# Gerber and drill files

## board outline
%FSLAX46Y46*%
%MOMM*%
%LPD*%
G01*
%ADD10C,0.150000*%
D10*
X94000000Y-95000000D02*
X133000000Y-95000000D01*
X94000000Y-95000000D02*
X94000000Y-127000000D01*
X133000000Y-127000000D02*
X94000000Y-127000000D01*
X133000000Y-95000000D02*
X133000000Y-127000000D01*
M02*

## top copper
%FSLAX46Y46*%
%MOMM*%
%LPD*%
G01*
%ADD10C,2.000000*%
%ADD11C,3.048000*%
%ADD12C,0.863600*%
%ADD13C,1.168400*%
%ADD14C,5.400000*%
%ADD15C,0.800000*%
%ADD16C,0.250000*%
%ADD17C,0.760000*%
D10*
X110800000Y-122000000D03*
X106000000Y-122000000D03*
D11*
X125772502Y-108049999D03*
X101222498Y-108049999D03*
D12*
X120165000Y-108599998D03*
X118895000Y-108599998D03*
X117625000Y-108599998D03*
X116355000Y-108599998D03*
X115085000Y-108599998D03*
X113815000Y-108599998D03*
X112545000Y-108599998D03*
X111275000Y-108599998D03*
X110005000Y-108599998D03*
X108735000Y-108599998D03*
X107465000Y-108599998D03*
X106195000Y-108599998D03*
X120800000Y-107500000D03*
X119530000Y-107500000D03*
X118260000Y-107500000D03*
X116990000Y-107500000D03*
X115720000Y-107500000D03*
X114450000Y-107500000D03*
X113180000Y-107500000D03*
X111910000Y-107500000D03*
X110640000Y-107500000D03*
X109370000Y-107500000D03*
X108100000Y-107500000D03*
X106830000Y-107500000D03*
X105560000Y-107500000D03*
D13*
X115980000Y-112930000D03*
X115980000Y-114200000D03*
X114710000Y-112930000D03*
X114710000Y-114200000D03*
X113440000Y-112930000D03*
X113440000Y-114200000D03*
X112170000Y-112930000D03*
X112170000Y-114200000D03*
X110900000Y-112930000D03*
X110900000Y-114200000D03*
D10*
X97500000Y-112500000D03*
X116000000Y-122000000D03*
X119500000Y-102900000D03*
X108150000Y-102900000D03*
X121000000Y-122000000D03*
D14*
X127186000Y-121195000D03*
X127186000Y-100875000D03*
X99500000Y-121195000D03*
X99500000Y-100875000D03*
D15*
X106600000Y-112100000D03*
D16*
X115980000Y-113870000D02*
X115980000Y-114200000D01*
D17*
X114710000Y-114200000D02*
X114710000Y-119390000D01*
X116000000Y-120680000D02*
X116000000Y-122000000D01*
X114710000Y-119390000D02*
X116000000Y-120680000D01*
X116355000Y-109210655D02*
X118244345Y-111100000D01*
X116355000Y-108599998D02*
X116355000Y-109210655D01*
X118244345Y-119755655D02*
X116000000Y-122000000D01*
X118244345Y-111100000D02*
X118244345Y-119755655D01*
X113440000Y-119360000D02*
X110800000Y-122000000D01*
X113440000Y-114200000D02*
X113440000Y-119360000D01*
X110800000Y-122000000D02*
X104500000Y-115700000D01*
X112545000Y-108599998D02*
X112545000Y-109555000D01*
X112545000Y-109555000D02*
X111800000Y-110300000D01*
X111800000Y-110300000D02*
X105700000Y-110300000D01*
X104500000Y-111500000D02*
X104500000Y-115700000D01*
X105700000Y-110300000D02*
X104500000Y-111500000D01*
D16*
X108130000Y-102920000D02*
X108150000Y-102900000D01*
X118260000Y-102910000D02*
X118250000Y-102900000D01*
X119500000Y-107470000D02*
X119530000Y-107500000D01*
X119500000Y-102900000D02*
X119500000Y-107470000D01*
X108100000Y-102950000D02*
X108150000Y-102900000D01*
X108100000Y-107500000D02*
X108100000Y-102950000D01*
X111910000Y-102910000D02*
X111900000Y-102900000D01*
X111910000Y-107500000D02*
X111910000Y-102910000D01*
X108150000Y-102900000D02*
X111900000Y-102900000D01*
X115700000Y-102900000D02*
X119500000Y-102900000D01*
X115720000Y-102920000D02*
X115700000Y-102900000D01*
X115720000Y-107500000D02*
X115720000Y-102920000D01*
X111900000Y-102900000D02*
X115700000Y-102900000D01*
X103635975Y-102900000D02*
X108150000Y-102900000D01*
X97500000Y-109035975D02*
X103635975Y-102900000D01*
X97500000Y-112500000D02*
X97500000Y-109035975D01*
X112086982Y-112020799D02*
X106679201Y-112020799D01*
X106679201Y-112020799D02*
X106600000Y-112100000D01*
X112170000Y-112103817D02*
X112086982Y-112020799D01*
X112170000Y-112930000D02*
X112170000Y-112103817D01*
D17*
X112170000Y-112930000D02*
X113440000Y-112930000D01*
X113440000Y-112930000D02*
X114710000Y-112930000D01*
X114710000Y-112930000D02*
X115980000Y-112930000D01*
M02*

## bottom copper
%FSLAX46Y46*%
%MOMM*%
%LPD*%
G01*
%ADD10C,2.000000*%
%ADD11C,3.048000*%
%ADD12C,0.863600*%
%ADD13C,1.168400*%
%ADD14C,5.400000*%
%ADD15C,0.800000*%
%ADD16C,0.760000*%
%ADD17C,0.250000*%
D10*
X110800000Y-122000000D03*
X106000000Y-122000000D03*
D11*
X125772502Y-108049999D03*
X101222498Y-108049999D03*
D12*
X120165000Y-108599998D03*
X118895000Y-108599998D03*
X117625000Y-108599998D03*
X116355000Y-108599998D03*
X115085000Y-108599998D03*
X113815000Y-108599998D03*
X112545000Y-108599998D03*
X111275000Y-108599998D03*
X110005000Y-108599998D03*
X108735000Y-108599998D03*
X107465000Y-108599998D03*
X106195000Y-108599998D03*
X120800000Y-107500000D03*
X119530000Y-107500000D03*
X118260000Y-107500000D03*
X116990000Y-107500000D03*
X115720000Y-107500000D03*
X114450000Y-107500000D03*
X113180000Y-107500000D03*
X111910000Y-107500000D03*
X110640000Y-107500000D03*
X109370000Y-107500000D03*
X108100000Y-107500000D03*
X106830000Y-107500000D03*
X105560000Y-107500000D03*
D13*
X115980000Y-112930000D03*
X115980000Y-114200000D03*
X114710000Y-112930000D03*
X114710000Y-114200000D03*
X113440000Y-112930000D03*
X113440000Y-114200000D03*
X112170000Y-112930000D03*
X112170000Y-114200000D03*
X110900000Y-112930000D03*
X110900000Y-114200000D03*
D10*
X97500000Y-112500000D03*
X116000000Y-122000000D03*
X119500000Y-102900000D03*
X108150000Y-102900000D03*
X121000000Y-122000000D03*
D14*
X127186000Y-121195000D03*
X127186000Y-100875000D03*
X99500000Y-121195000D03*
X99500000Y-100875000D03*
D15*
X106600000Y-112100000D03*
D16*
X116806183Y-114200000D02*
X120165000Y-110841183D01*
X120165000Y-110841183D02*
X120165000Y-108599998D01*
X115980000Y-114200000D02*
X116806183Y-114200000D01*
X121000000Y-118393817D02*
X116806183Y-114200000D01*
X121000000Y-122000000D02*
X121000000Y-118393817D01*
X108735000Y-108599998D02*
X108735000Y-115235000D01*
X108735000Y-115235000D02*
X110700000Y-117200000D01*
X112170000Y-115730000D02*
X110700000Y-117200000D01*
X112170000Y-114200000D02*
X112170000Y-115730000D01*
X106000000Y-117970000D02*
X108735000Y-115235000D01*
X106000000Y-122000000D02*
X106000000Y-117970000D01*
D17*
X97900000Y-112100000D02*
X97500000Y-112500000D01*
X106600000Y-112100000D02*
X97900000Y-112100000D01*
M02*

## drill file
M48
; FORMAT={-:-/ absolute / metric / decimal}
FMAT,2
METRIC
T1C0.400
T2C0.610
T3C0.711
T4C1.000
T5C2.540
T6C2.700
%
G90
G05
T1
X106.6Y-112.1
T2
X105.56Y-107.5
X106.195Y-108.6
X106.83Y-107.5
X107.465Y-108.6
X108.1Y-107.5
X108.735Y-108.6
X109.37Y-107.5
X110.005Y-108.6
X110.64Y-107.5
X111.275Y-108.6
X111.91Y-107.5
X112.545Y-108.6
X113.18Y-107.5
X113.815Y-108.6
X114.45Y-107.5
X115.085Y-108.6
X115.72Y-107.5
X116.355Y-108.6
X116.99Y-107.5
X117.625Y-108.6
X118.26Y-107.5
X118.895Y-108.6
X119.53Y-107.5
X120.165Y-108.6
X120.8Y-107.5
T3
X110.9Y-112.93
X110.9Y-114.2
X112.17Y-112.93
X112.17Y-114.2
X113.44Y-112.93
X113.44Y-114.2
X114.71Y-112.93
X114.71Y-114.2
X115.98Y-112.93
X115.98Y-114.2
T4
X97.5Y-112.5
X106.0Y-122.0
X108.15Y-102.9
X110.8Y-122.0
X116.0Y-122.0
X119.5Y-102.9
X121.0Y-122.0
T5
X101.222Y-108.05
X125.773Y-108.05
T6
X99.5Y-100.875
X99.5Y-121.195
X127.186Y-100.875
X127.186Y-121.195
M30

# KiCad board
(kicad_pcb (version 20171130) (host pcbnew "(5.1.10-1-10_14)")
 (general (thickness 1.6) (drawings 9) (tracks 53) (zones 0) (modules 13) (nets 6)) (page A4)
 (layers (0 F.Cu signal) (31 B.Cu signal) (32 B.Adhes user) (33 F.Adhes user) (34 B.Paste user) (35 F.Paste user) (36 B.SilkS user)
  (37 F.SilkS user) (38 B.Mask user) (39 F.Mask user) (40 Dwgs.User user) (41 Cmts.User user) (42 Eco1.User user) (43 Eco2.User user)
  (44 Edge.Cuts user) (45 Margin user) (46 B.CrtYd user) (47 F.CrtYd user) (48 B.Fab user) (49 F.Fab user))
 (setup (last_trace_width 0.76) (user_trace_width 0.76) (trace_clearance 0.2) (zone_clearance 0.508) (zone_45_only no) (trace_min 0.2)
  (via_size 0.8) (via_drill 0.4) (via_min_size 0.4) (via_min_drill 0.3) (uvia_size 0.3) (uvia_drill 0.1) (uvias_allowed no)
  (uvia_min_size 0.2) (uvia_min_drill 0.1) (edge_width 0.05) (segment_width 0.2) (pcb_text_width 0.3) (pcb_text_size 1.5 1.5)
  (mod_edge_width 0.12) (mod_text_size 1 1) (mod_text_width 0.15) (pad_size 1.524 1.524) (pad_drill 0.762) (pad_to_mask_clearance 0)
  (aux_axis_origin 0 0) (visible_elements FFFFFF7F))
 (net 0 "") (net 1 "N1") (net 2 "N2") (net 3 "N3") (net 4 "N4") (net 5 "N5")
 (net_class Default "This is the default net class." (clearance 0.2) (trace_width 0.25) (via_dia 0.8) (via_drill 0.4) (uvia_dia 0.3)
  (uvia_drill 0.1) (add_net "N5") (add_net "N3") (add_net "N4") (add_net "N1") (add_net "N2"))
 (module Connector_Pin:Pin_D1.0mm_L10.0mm (layer F.Cu) (at 110.8 122)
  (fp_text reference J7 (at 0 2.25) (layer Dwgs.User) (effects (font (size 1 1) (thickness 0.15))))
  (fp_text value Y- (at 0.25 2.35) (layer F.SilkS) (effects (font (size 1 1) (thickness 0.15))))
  (pad 1 thru_hole circle (at 0 0) (size 2 2) (drill 1) (layers *.Cu *.Mask) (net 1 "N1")))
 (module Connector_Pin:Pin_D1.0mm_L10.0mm (layer F.Cu) (at 106 122)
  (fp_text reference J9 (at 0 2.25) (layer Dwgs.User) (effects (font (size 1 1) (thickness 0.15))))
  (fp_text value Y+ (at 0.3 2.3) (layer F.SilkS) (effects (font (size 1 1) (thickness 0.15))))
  (pad 1 thru_hole circle (at 0 0) (size 2 2) (drill 1) (layers *.Cu *.Mask) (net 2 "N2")))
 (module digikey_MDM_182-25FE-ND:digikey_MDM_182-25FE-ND (layer F.Cu) (at 120.8 107.5)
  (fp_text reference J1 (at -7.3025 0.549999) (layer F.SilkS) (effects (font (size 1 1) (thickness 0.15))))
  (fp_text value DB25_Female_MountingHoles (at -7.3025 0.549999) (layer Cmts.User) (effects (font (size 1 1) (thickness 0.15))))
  (pad 28 thru_hole circle (at 4.972502 0.549999 90) (size 3.048 3.048) (drill 2.54) (layers *.Cu *.Mask))
  (pad 27 thru_hole circle (at -19.577502 0.549999 90) (size 3.048 3.048) (drill 2.54) (layers *.Cu *.Mask))
  (pad 14 thru_hole circle (at -0.635 1.099998) (size 0.8636 0.8636) (drill 0.6096) (layers *.Cu *.Mask) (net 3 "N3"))
  (pad 15 thru_hole circle (at -1.905 1.099998) (size 0.8636 0.8636) (drill 0.6096) (layers *.Cu *.Mask))
  (pad 16 thru_hole circle (at -3.175 1.099998) (size 0.8636 0.8636) (drill 0.6096) (layers *.Cu *.Mask))
  (pad 17 thru_hole circle (at -4.445 1.099998) (size 0.8636 0.8636) (drill 0.6096) (layers *.Cu *.Mask) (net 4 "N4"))
  (pad 18 thru_hole circle (at -5.715 1.099998) (size 0.8636 0.8636) (drill 0.6096) (layers *.Cu *.Mask))
  (pad 19 thru_hole circle (at -6.985 1.099998) (size 0.8636 0.8636) (drill 0.6096) (layers *.Cu *.Mask))
  (pad 20 thru_hole circle (at -8.255 1.099998) (size 0.8636 0.8636) (drill 0.6096) (layers *.Cu *.Mask) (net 1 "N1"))
  (pad 21 thru_hole circle (at -9.525 1.099998) (size 0.8636 0.8636) (drill 0.6096) (layers *.Cu *.Mask))
  (pad 22 thru_hole circle (at -10.795 1.099998) (size 0.8636 0.8636) (drill 0.6096) (layers *.Cu *.Mask))
  (pad 23 thru_hole circle (at -12.065 1.099998) (size 0.8636 0.8636) (drill 0.6096) (layers *.Cu *.Mask) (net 2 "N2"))
  (pad 24 thru_hole circle (at -13.335 1.099998) (size 0.8636 0.8636) (drill 0.6096) (layers *.Cu *.Mask))
  (pad 25 thru_hole circle (at -14.605 1.099998) (size 0.8636 0.8636) (drill 0.6096) (layers *.Cu *.Mask))
  (pad 1 thru_hole circle (at 0 0) (size 0.8636 0.8636) (drill 0.6096) (layers *.Cu *.Mask))
  (pad 2 thru_hole circle (at -1.27 0) (size 0.8636 0.8636) (drill 0.6096) (layers *.Cu *.Mask) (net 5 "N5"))
  (pad 3 thru_hole circle (at -2.54 0) (size 0.8636 0.8636) (drill 0.6096) (layers *.Cu *.Mask))
  (pad 4 thru_hole circle (at -3.81 0) (size 0.8636 0.8636) (drill 0.6096) (layers *.Cu *.Mask))
  (pad 5 thru_hole circle (at -5.08 0) (size 0.8636 0.8636) (drill 0.6096) (layers *.Cu *.Mask) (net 5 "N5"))
  (pad 6 thru_hole circle (at -6.35 0) (size 0.8636 0.8636) (drill 0.6096) (layers *.Cu *.Mask))
  (pad 7 thru_hole circle (at -7.62 0) (size 0.8636 0.8636) (drill 0.6096) (layers *.Cu *.Mask))
  (pad 8 thru_hole circle (at -8.89 0) (size 0.8636 0.8636) (drill 0.6096) (layers *.Cu *.Mask) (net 5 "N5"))
  (pad 9 thru_hole circle (at -10.16 0) (size 0.8636 0.8636) (drill 0.6096) (layers *.Cu *.Mask))
  (pad 10 thru_hole circle (at -11.43 0) (size 0.8636 0.8636) (drill 0.6096) (layers *.Cu *.Mask))
  (pad 11 thru_hole circle (at -12.7 0) (size 0.8636 0.8636) (drill 0.6096) (layers *.Cu *.Mask) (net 5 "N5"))
  (pad 12 thru_hole circle (at -13.97 0) (size 0.8636 0.8636) (drill 0.6096) (layers *.Cu *.Mask))
  (pad 13 thru_hole circle (at -15.24 0) (size 0.8636 0.8636) (drill 0.6096) (layers *.Cu *.Mask)))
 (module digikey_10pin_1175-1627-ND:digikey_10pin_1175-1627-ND (layer F.Cu) (at 110.9 114.2)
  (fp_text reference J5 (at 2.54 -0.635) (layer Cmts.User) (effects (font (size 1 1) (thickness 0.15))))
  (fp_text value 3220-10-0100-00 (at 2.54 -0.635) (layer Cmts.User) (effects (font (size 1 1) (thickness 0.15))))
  (pad 10 thru_hole circle (at 5.08 -1.27) (size 1.1684 1.1684) (drill 0.7112) (layers *.Cu *.Mask) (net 5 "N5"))
  (pad 9 thru_hole circle (at 5.08 0) (size 1.1684 1.1684) (drill 0.7112) (layers *.Cu *.Mask) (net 3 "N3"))
  (pad 8 thru_hole circle (at 3.81 -1.27) (size 1.1684 1.1684) (drill 0.7112) (layers *.Cu *.Mask) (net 5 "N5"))
  (pad 7 thru_hole circle (at 3.81 0) (size 1.1684 1.1684) (drill 0.7112) (layers *.Cu *.Mask) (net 4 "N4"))
  (pad 6 thru_hole circle (at 2.54 -1.27) (size 1.1684 1.1684) (drill 0.7112) (layers *.Cu *.Mask) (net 5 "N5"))
  (pad 5 thru_hole circle (at 2.54 0) (size 1.1684 1.1684) (drill 0.7112) (layers *.Cu *.Mask) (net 1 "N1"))
  (pad 4 thru_hole circle (at 1.27 -1.27) (size 1.1684 1.1684) (drill 0.7112) (layers *.Cu *.Mask) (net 5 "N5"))
  (pad 3 thru_hole circle (at 1.27 0) (size 1.1684 1.1684) (drill 0.7112) (layers *.Cu *.Mask) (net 2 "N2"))
  (pad 2 thru_hole circle (at 0 -1.27) (size 1.1684 1.1684) (drill 0.7112) (layers *.Cu *.Mask))
  (pad 1 thru_hole circle (at 0 0) (size 1.1684 1.1684) (drill 0.7112) (layers *.Cu *.Mask)))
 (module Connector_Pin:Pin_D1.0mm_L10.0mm (layer F.Cu) (at 97.5 112.5)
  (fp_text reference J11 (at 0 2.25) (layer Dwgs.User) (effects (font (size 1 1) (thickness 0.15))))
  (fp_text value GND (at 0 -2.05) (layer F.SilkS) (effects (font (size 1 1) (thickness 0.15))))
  (pad 1 thru_hole circle (at 0 0) (size 2 2) (drill 1) (layers *.Cu *.Mask) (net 5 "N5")))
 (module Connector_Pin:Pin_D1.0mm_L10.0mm (layer F.Cu) (at 116 122)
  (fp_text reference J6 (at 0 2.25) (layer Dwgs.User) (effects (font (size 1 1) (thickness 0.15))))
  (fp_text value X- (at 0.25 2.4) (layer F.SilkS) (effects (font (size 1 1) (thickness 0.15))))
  (pad 1 thru_hole circle (at 0 0) (size 2 2) (drill 1) (layers *.Cu *.Mask) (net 4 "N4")))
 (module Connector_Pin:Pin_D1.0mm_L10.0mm (layer F.Cu) (at 119.5 102.9)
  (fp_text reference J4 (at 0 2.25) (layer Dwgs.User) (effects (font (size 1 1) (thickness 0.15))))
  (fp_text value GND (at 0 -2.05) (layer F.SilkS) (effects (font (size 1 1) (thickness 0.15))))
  (pad 1 thru_hole circle (at 0 0) (size 2 2) (drill 1) (layers *.Cu *.Mask) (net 5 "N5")))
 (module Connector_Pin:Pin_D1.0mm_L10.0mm (layer F.Cu) (at 108.15 102.9)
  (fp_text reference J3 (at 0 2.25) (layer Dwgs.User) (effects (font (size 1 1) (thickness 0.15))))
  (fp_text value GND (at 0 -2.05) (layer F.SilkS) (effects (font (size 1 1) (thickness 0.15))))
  (pad 1 thru_hole circle (at 0 0) (size 2 2) (drill 1) (layers *.Cu *.Mask) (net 5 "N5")))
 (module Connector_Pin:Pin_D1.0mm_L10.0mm (layer F.Cu) (at 121 122)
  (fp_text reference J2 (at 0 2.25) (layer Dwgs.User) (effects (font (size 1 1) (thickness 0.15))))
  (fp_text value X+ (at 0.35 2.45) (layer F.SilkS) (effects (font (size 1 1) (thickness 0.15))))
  (pad 1 thru_hole circle (at 0 0) (size 2 2) (drill 1) (layers *.Cu *.Mask) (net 3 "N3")))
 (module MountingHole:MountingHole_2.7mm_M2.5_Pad (layer F.Cu) (at 127.186 121.195)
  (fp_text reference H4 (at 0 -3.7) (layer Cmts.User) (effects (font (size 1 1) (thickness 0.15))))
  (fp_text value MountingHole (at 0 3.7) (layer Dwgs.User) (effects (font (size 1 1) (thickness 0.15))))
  (pad 1 thru_hole circle (at 0 0) (size 5.4 5.4) (drill 2.7) (layers *.Cu *.Mask)))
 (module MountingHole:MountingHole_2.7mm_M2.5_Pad (layer F.Cu) (at 127.186 100.875)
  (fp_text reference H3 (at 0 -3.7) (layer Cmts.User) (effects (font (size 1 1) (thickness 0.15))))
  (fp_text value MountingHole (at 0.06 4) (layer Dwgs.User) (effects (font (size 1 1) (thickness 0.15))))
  (pad 1 thru_hole circle (at 0 0) (size 5.4 5.4) (drill 2.7) (layers *.Cu *.Mask)))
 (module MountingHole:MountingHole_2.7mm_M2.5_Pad (layer F.Cu) (at 99.5 121.195)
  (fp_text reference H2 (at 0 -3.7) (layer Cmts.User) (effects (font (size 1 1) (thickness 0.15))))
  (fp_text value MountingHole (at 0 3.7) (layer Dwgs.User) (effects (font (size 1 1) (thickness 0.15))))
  (pad 1 thru_hole circle (at 0 0) (size 5.4 5.4) (drill 2.7) (layers *.Cu *.Mask)))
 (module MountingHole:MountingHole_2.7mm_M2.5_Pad (layer F.Cu) (at 99.5 100.875)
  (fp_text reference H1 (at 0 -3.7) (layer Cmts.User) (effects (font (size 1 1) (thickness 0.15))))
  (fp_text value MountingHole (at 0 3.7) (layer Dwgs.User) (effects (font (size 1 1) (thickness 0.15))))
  (pad 1 thru_hole circle (at 0 0) (size 5.4 5.4) (drill 2.7) (layers *.Cu *.Mask)))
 (gr_line (start 94 95) (end 133 95) (layer Edge.Cuts) (width 0.15))
 (gr_line (start 94 95) (end 94 127) (layer Edge.Cuts) (width 0.15))
 (gr_line (start 133 127) (end 94 127) (layer Edge.Cuts) (width 0.15))
 (gr_line (start 133 95) (end 133 127) (layer Edge.Cuts) (width 0.15))
 (segment (start 115.98 113.87) (end 115.98 114.2) (width 0.25) (layer F.Cu) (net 3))
 (segment (start 116.806183 114.2) (end 120.165 110.841183) (width 0.76) (layer B.Cu) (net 3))
 (segment (start 120.165 110.841183) (end 120.165 108.599998) (width 0.76) (layer B.Cu) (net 3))
 (segment (start 115.98 114.2) (end 116.806183 114.2) (width 0.76) (layer B.Cu) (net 3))
 (segment (start 121 118.393817) (end 116.806183 114.2) (width 0.76) (layer B.Cu) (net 3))
 (segment (start 121 122) (end 121 118.393817) (width 0.76) (layer B.Cu) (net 3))
 (segment (start 114.71 114.2) (end 114.71 119.39) (width 0.76) (layer F.Cu) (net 4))
 (segment (start 116 120.68) (end 116 122) (width 0.76) (layer F.Cu) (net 4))
 (segment (start 114.71 119.39) (end 116 120.68) (width 0.76) (layer F.Cu) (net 4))
 (segment (start 116.355 109.210655) (end 118.244345 111.1) (width 0.76) (layer F.Cu) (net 4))
 (segment (start 116.355 108.599998) (end 116.355 109.210655) (width 0.76) (layer F.Cu) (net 4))
 (segment (start 118.244345 119.755655) (end 116 122) (width 0.76) (layer F.Cu) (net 4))
 (segment (start 118.244345 111.1) (end 118.244345 119.755655) (width 0.76) (layer F.Cu) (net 4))
 (segment (start 113.44 119.36) (end 110.8 122) (width 0.76) (layer F.Cu) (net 1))
 (segment (start 113.44 114.2) (end 113.44 119.36) (width 0.76) (layer F.Cu) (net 1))
 (segment (start 110.8 122) (end 104.5 115.7) (width 0.76) (layer F.Cu) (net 1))
 (segment (start 112.545 108.599998) (end 112.545 109.555) (width 0.76) (layer F.Cu) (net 1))
 (segment (start 112.545 109.555) (end 111.8 110.3) (width 0.76) (layer F.Cu) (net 1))
 (segment (start 111.8 110.3) (end 105.7 110.3) (width 0.76) (layer F.Cu) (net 1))
 (segment (start 104.5 111.5) (end 104.5 115.7) (width 0.76) (layer F.Cu) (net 1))
 (segment (start 105.7 110.3) (end 104.5 111.5) (width 0.76) (layer F.Cu) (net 1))
 (segment (start 108.735 108.599998) (end 108.735 115.235) (width 0.76) (layer B.Cu) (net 2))
 (segment (start 108.735 115.235) (end 110.7 117.2) (width 0.76) (layer B.Cu) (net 2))
 (segment (start 112.17 115.73) (end 110.7 117.2) (width 0.76) (layer B.Cu) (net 2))
 (segment (start 112.17 114.2) (end 112.17 115.73) (width 0.76) (layer B.Cu) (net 2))
 (segment (start 106 117.97) (end 108.735 115.235) (width 0.76) (layer B.Cu) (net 2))
 (segment (start 106 122) (end 106 117.97) (width 0.76) (layer B.Cu) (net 2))
 (segment (start 108.13 102.92) (end 108.15 102.9) (width 0.25) (layer F.Cu) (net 5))
 (segment (start 118.26 102.91) (end 118.25 102.9) (width 0.25) (layer F.Cu) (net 5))
 (segment (start 119.5 107.47) (end 119.53 107.5) (width 0.25) (layer F.Cu) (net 5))
 (segment (start 119.5 102.9) (end 119.5 107.47) (width 0.25) (layer F.Cu) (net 5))
 (segment (start 108.1 102.95) (end 108.15 102.9) (width 0.25) (layer F.Cu) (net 5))
 (segment (start 108.1 107.5) (end 108.1 102.95) (width 0.25) (layer F.Cu) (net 5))
 (segment (start 111.91 102.91) (end 111.9 102.9) (width 0.25) (layer F.Cu) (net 5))
 (segment (start 111.91 107.5) (end 111.91 102.91) (width 0.25) (layer F.Cu) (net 5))
 (segment (start 108.15 102.9) (end 111.9 102.9) (width 0.25) (layer F.Cu) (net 5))
 (segment (start 115.7 102.9) (end 119.5 102.9) (width 0.25) (layer F.Cu) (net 5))
 (segment (start 115.72 102.92) (end 115.7 102.9) (width 0.25) (layer F.Cu) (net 5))
 (segment (start 115.72 107.5) (end 115.72 102.92) (width 0.25) (layer F.Cu) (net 5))
 (segment (start 111.9 102.9) (end 115.7 102.9) (width 0.25) (layer F.Cu) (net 5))
 (segment (start 103.635975 102.9) (end 108.15 102.9) (width 0.25) (layer F.Cu) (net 5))
 (segment (start 97.5 109.035975) (end 103.635975 102.9) (width 0.25) (layer F.Cu) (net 5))
 (segment (start 97.5 112.5) (end 97.5 109.035975) (width 0.25) (layer F.Cu) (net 5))
 (via (at 106.6 112.1) (size 0.8) (drill 0.4) (layers F.Cu B.Cu) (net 5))
 (segment (start 112.086982 112.020799) (end 106.679201 112.020799) (width 0.25) (layer F.Cu) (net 5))
 (segment (start 106.679201 112.020799) (end 106.6 112.1) (width 0.25) (layer F.Cu) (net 5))
 (segment (start 112.17 112.103817) (end 112.086982 112.020799) (width 0.25) (layer F.Cu) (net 5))
 (segment (start 112.17 112.93) (end 112.17 112.103817) (width 0.25) (layer F.Cu) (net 5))
 (segment (start 97.9 112.1) (end 97.5 112.5) (width 0.25) (layer B.Cu) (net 5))
 (segment (start 106.6 112.1) (end 97.9 112.1) (width 0.25) (layer B.Cu) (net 5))
 (segment (start 112.17 112.93) (end 113.44 112.93) (width 0.76) (layer F.Cu) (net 5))
 (segment (start 113.44 112.93) (end 114.71 112.93) (width 0.76) (layer F.Cu) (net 5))
 (segment (start 114.71 112.93) (end 115.98 112.93) (width 0.76) (layer F.Cu) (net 5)))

